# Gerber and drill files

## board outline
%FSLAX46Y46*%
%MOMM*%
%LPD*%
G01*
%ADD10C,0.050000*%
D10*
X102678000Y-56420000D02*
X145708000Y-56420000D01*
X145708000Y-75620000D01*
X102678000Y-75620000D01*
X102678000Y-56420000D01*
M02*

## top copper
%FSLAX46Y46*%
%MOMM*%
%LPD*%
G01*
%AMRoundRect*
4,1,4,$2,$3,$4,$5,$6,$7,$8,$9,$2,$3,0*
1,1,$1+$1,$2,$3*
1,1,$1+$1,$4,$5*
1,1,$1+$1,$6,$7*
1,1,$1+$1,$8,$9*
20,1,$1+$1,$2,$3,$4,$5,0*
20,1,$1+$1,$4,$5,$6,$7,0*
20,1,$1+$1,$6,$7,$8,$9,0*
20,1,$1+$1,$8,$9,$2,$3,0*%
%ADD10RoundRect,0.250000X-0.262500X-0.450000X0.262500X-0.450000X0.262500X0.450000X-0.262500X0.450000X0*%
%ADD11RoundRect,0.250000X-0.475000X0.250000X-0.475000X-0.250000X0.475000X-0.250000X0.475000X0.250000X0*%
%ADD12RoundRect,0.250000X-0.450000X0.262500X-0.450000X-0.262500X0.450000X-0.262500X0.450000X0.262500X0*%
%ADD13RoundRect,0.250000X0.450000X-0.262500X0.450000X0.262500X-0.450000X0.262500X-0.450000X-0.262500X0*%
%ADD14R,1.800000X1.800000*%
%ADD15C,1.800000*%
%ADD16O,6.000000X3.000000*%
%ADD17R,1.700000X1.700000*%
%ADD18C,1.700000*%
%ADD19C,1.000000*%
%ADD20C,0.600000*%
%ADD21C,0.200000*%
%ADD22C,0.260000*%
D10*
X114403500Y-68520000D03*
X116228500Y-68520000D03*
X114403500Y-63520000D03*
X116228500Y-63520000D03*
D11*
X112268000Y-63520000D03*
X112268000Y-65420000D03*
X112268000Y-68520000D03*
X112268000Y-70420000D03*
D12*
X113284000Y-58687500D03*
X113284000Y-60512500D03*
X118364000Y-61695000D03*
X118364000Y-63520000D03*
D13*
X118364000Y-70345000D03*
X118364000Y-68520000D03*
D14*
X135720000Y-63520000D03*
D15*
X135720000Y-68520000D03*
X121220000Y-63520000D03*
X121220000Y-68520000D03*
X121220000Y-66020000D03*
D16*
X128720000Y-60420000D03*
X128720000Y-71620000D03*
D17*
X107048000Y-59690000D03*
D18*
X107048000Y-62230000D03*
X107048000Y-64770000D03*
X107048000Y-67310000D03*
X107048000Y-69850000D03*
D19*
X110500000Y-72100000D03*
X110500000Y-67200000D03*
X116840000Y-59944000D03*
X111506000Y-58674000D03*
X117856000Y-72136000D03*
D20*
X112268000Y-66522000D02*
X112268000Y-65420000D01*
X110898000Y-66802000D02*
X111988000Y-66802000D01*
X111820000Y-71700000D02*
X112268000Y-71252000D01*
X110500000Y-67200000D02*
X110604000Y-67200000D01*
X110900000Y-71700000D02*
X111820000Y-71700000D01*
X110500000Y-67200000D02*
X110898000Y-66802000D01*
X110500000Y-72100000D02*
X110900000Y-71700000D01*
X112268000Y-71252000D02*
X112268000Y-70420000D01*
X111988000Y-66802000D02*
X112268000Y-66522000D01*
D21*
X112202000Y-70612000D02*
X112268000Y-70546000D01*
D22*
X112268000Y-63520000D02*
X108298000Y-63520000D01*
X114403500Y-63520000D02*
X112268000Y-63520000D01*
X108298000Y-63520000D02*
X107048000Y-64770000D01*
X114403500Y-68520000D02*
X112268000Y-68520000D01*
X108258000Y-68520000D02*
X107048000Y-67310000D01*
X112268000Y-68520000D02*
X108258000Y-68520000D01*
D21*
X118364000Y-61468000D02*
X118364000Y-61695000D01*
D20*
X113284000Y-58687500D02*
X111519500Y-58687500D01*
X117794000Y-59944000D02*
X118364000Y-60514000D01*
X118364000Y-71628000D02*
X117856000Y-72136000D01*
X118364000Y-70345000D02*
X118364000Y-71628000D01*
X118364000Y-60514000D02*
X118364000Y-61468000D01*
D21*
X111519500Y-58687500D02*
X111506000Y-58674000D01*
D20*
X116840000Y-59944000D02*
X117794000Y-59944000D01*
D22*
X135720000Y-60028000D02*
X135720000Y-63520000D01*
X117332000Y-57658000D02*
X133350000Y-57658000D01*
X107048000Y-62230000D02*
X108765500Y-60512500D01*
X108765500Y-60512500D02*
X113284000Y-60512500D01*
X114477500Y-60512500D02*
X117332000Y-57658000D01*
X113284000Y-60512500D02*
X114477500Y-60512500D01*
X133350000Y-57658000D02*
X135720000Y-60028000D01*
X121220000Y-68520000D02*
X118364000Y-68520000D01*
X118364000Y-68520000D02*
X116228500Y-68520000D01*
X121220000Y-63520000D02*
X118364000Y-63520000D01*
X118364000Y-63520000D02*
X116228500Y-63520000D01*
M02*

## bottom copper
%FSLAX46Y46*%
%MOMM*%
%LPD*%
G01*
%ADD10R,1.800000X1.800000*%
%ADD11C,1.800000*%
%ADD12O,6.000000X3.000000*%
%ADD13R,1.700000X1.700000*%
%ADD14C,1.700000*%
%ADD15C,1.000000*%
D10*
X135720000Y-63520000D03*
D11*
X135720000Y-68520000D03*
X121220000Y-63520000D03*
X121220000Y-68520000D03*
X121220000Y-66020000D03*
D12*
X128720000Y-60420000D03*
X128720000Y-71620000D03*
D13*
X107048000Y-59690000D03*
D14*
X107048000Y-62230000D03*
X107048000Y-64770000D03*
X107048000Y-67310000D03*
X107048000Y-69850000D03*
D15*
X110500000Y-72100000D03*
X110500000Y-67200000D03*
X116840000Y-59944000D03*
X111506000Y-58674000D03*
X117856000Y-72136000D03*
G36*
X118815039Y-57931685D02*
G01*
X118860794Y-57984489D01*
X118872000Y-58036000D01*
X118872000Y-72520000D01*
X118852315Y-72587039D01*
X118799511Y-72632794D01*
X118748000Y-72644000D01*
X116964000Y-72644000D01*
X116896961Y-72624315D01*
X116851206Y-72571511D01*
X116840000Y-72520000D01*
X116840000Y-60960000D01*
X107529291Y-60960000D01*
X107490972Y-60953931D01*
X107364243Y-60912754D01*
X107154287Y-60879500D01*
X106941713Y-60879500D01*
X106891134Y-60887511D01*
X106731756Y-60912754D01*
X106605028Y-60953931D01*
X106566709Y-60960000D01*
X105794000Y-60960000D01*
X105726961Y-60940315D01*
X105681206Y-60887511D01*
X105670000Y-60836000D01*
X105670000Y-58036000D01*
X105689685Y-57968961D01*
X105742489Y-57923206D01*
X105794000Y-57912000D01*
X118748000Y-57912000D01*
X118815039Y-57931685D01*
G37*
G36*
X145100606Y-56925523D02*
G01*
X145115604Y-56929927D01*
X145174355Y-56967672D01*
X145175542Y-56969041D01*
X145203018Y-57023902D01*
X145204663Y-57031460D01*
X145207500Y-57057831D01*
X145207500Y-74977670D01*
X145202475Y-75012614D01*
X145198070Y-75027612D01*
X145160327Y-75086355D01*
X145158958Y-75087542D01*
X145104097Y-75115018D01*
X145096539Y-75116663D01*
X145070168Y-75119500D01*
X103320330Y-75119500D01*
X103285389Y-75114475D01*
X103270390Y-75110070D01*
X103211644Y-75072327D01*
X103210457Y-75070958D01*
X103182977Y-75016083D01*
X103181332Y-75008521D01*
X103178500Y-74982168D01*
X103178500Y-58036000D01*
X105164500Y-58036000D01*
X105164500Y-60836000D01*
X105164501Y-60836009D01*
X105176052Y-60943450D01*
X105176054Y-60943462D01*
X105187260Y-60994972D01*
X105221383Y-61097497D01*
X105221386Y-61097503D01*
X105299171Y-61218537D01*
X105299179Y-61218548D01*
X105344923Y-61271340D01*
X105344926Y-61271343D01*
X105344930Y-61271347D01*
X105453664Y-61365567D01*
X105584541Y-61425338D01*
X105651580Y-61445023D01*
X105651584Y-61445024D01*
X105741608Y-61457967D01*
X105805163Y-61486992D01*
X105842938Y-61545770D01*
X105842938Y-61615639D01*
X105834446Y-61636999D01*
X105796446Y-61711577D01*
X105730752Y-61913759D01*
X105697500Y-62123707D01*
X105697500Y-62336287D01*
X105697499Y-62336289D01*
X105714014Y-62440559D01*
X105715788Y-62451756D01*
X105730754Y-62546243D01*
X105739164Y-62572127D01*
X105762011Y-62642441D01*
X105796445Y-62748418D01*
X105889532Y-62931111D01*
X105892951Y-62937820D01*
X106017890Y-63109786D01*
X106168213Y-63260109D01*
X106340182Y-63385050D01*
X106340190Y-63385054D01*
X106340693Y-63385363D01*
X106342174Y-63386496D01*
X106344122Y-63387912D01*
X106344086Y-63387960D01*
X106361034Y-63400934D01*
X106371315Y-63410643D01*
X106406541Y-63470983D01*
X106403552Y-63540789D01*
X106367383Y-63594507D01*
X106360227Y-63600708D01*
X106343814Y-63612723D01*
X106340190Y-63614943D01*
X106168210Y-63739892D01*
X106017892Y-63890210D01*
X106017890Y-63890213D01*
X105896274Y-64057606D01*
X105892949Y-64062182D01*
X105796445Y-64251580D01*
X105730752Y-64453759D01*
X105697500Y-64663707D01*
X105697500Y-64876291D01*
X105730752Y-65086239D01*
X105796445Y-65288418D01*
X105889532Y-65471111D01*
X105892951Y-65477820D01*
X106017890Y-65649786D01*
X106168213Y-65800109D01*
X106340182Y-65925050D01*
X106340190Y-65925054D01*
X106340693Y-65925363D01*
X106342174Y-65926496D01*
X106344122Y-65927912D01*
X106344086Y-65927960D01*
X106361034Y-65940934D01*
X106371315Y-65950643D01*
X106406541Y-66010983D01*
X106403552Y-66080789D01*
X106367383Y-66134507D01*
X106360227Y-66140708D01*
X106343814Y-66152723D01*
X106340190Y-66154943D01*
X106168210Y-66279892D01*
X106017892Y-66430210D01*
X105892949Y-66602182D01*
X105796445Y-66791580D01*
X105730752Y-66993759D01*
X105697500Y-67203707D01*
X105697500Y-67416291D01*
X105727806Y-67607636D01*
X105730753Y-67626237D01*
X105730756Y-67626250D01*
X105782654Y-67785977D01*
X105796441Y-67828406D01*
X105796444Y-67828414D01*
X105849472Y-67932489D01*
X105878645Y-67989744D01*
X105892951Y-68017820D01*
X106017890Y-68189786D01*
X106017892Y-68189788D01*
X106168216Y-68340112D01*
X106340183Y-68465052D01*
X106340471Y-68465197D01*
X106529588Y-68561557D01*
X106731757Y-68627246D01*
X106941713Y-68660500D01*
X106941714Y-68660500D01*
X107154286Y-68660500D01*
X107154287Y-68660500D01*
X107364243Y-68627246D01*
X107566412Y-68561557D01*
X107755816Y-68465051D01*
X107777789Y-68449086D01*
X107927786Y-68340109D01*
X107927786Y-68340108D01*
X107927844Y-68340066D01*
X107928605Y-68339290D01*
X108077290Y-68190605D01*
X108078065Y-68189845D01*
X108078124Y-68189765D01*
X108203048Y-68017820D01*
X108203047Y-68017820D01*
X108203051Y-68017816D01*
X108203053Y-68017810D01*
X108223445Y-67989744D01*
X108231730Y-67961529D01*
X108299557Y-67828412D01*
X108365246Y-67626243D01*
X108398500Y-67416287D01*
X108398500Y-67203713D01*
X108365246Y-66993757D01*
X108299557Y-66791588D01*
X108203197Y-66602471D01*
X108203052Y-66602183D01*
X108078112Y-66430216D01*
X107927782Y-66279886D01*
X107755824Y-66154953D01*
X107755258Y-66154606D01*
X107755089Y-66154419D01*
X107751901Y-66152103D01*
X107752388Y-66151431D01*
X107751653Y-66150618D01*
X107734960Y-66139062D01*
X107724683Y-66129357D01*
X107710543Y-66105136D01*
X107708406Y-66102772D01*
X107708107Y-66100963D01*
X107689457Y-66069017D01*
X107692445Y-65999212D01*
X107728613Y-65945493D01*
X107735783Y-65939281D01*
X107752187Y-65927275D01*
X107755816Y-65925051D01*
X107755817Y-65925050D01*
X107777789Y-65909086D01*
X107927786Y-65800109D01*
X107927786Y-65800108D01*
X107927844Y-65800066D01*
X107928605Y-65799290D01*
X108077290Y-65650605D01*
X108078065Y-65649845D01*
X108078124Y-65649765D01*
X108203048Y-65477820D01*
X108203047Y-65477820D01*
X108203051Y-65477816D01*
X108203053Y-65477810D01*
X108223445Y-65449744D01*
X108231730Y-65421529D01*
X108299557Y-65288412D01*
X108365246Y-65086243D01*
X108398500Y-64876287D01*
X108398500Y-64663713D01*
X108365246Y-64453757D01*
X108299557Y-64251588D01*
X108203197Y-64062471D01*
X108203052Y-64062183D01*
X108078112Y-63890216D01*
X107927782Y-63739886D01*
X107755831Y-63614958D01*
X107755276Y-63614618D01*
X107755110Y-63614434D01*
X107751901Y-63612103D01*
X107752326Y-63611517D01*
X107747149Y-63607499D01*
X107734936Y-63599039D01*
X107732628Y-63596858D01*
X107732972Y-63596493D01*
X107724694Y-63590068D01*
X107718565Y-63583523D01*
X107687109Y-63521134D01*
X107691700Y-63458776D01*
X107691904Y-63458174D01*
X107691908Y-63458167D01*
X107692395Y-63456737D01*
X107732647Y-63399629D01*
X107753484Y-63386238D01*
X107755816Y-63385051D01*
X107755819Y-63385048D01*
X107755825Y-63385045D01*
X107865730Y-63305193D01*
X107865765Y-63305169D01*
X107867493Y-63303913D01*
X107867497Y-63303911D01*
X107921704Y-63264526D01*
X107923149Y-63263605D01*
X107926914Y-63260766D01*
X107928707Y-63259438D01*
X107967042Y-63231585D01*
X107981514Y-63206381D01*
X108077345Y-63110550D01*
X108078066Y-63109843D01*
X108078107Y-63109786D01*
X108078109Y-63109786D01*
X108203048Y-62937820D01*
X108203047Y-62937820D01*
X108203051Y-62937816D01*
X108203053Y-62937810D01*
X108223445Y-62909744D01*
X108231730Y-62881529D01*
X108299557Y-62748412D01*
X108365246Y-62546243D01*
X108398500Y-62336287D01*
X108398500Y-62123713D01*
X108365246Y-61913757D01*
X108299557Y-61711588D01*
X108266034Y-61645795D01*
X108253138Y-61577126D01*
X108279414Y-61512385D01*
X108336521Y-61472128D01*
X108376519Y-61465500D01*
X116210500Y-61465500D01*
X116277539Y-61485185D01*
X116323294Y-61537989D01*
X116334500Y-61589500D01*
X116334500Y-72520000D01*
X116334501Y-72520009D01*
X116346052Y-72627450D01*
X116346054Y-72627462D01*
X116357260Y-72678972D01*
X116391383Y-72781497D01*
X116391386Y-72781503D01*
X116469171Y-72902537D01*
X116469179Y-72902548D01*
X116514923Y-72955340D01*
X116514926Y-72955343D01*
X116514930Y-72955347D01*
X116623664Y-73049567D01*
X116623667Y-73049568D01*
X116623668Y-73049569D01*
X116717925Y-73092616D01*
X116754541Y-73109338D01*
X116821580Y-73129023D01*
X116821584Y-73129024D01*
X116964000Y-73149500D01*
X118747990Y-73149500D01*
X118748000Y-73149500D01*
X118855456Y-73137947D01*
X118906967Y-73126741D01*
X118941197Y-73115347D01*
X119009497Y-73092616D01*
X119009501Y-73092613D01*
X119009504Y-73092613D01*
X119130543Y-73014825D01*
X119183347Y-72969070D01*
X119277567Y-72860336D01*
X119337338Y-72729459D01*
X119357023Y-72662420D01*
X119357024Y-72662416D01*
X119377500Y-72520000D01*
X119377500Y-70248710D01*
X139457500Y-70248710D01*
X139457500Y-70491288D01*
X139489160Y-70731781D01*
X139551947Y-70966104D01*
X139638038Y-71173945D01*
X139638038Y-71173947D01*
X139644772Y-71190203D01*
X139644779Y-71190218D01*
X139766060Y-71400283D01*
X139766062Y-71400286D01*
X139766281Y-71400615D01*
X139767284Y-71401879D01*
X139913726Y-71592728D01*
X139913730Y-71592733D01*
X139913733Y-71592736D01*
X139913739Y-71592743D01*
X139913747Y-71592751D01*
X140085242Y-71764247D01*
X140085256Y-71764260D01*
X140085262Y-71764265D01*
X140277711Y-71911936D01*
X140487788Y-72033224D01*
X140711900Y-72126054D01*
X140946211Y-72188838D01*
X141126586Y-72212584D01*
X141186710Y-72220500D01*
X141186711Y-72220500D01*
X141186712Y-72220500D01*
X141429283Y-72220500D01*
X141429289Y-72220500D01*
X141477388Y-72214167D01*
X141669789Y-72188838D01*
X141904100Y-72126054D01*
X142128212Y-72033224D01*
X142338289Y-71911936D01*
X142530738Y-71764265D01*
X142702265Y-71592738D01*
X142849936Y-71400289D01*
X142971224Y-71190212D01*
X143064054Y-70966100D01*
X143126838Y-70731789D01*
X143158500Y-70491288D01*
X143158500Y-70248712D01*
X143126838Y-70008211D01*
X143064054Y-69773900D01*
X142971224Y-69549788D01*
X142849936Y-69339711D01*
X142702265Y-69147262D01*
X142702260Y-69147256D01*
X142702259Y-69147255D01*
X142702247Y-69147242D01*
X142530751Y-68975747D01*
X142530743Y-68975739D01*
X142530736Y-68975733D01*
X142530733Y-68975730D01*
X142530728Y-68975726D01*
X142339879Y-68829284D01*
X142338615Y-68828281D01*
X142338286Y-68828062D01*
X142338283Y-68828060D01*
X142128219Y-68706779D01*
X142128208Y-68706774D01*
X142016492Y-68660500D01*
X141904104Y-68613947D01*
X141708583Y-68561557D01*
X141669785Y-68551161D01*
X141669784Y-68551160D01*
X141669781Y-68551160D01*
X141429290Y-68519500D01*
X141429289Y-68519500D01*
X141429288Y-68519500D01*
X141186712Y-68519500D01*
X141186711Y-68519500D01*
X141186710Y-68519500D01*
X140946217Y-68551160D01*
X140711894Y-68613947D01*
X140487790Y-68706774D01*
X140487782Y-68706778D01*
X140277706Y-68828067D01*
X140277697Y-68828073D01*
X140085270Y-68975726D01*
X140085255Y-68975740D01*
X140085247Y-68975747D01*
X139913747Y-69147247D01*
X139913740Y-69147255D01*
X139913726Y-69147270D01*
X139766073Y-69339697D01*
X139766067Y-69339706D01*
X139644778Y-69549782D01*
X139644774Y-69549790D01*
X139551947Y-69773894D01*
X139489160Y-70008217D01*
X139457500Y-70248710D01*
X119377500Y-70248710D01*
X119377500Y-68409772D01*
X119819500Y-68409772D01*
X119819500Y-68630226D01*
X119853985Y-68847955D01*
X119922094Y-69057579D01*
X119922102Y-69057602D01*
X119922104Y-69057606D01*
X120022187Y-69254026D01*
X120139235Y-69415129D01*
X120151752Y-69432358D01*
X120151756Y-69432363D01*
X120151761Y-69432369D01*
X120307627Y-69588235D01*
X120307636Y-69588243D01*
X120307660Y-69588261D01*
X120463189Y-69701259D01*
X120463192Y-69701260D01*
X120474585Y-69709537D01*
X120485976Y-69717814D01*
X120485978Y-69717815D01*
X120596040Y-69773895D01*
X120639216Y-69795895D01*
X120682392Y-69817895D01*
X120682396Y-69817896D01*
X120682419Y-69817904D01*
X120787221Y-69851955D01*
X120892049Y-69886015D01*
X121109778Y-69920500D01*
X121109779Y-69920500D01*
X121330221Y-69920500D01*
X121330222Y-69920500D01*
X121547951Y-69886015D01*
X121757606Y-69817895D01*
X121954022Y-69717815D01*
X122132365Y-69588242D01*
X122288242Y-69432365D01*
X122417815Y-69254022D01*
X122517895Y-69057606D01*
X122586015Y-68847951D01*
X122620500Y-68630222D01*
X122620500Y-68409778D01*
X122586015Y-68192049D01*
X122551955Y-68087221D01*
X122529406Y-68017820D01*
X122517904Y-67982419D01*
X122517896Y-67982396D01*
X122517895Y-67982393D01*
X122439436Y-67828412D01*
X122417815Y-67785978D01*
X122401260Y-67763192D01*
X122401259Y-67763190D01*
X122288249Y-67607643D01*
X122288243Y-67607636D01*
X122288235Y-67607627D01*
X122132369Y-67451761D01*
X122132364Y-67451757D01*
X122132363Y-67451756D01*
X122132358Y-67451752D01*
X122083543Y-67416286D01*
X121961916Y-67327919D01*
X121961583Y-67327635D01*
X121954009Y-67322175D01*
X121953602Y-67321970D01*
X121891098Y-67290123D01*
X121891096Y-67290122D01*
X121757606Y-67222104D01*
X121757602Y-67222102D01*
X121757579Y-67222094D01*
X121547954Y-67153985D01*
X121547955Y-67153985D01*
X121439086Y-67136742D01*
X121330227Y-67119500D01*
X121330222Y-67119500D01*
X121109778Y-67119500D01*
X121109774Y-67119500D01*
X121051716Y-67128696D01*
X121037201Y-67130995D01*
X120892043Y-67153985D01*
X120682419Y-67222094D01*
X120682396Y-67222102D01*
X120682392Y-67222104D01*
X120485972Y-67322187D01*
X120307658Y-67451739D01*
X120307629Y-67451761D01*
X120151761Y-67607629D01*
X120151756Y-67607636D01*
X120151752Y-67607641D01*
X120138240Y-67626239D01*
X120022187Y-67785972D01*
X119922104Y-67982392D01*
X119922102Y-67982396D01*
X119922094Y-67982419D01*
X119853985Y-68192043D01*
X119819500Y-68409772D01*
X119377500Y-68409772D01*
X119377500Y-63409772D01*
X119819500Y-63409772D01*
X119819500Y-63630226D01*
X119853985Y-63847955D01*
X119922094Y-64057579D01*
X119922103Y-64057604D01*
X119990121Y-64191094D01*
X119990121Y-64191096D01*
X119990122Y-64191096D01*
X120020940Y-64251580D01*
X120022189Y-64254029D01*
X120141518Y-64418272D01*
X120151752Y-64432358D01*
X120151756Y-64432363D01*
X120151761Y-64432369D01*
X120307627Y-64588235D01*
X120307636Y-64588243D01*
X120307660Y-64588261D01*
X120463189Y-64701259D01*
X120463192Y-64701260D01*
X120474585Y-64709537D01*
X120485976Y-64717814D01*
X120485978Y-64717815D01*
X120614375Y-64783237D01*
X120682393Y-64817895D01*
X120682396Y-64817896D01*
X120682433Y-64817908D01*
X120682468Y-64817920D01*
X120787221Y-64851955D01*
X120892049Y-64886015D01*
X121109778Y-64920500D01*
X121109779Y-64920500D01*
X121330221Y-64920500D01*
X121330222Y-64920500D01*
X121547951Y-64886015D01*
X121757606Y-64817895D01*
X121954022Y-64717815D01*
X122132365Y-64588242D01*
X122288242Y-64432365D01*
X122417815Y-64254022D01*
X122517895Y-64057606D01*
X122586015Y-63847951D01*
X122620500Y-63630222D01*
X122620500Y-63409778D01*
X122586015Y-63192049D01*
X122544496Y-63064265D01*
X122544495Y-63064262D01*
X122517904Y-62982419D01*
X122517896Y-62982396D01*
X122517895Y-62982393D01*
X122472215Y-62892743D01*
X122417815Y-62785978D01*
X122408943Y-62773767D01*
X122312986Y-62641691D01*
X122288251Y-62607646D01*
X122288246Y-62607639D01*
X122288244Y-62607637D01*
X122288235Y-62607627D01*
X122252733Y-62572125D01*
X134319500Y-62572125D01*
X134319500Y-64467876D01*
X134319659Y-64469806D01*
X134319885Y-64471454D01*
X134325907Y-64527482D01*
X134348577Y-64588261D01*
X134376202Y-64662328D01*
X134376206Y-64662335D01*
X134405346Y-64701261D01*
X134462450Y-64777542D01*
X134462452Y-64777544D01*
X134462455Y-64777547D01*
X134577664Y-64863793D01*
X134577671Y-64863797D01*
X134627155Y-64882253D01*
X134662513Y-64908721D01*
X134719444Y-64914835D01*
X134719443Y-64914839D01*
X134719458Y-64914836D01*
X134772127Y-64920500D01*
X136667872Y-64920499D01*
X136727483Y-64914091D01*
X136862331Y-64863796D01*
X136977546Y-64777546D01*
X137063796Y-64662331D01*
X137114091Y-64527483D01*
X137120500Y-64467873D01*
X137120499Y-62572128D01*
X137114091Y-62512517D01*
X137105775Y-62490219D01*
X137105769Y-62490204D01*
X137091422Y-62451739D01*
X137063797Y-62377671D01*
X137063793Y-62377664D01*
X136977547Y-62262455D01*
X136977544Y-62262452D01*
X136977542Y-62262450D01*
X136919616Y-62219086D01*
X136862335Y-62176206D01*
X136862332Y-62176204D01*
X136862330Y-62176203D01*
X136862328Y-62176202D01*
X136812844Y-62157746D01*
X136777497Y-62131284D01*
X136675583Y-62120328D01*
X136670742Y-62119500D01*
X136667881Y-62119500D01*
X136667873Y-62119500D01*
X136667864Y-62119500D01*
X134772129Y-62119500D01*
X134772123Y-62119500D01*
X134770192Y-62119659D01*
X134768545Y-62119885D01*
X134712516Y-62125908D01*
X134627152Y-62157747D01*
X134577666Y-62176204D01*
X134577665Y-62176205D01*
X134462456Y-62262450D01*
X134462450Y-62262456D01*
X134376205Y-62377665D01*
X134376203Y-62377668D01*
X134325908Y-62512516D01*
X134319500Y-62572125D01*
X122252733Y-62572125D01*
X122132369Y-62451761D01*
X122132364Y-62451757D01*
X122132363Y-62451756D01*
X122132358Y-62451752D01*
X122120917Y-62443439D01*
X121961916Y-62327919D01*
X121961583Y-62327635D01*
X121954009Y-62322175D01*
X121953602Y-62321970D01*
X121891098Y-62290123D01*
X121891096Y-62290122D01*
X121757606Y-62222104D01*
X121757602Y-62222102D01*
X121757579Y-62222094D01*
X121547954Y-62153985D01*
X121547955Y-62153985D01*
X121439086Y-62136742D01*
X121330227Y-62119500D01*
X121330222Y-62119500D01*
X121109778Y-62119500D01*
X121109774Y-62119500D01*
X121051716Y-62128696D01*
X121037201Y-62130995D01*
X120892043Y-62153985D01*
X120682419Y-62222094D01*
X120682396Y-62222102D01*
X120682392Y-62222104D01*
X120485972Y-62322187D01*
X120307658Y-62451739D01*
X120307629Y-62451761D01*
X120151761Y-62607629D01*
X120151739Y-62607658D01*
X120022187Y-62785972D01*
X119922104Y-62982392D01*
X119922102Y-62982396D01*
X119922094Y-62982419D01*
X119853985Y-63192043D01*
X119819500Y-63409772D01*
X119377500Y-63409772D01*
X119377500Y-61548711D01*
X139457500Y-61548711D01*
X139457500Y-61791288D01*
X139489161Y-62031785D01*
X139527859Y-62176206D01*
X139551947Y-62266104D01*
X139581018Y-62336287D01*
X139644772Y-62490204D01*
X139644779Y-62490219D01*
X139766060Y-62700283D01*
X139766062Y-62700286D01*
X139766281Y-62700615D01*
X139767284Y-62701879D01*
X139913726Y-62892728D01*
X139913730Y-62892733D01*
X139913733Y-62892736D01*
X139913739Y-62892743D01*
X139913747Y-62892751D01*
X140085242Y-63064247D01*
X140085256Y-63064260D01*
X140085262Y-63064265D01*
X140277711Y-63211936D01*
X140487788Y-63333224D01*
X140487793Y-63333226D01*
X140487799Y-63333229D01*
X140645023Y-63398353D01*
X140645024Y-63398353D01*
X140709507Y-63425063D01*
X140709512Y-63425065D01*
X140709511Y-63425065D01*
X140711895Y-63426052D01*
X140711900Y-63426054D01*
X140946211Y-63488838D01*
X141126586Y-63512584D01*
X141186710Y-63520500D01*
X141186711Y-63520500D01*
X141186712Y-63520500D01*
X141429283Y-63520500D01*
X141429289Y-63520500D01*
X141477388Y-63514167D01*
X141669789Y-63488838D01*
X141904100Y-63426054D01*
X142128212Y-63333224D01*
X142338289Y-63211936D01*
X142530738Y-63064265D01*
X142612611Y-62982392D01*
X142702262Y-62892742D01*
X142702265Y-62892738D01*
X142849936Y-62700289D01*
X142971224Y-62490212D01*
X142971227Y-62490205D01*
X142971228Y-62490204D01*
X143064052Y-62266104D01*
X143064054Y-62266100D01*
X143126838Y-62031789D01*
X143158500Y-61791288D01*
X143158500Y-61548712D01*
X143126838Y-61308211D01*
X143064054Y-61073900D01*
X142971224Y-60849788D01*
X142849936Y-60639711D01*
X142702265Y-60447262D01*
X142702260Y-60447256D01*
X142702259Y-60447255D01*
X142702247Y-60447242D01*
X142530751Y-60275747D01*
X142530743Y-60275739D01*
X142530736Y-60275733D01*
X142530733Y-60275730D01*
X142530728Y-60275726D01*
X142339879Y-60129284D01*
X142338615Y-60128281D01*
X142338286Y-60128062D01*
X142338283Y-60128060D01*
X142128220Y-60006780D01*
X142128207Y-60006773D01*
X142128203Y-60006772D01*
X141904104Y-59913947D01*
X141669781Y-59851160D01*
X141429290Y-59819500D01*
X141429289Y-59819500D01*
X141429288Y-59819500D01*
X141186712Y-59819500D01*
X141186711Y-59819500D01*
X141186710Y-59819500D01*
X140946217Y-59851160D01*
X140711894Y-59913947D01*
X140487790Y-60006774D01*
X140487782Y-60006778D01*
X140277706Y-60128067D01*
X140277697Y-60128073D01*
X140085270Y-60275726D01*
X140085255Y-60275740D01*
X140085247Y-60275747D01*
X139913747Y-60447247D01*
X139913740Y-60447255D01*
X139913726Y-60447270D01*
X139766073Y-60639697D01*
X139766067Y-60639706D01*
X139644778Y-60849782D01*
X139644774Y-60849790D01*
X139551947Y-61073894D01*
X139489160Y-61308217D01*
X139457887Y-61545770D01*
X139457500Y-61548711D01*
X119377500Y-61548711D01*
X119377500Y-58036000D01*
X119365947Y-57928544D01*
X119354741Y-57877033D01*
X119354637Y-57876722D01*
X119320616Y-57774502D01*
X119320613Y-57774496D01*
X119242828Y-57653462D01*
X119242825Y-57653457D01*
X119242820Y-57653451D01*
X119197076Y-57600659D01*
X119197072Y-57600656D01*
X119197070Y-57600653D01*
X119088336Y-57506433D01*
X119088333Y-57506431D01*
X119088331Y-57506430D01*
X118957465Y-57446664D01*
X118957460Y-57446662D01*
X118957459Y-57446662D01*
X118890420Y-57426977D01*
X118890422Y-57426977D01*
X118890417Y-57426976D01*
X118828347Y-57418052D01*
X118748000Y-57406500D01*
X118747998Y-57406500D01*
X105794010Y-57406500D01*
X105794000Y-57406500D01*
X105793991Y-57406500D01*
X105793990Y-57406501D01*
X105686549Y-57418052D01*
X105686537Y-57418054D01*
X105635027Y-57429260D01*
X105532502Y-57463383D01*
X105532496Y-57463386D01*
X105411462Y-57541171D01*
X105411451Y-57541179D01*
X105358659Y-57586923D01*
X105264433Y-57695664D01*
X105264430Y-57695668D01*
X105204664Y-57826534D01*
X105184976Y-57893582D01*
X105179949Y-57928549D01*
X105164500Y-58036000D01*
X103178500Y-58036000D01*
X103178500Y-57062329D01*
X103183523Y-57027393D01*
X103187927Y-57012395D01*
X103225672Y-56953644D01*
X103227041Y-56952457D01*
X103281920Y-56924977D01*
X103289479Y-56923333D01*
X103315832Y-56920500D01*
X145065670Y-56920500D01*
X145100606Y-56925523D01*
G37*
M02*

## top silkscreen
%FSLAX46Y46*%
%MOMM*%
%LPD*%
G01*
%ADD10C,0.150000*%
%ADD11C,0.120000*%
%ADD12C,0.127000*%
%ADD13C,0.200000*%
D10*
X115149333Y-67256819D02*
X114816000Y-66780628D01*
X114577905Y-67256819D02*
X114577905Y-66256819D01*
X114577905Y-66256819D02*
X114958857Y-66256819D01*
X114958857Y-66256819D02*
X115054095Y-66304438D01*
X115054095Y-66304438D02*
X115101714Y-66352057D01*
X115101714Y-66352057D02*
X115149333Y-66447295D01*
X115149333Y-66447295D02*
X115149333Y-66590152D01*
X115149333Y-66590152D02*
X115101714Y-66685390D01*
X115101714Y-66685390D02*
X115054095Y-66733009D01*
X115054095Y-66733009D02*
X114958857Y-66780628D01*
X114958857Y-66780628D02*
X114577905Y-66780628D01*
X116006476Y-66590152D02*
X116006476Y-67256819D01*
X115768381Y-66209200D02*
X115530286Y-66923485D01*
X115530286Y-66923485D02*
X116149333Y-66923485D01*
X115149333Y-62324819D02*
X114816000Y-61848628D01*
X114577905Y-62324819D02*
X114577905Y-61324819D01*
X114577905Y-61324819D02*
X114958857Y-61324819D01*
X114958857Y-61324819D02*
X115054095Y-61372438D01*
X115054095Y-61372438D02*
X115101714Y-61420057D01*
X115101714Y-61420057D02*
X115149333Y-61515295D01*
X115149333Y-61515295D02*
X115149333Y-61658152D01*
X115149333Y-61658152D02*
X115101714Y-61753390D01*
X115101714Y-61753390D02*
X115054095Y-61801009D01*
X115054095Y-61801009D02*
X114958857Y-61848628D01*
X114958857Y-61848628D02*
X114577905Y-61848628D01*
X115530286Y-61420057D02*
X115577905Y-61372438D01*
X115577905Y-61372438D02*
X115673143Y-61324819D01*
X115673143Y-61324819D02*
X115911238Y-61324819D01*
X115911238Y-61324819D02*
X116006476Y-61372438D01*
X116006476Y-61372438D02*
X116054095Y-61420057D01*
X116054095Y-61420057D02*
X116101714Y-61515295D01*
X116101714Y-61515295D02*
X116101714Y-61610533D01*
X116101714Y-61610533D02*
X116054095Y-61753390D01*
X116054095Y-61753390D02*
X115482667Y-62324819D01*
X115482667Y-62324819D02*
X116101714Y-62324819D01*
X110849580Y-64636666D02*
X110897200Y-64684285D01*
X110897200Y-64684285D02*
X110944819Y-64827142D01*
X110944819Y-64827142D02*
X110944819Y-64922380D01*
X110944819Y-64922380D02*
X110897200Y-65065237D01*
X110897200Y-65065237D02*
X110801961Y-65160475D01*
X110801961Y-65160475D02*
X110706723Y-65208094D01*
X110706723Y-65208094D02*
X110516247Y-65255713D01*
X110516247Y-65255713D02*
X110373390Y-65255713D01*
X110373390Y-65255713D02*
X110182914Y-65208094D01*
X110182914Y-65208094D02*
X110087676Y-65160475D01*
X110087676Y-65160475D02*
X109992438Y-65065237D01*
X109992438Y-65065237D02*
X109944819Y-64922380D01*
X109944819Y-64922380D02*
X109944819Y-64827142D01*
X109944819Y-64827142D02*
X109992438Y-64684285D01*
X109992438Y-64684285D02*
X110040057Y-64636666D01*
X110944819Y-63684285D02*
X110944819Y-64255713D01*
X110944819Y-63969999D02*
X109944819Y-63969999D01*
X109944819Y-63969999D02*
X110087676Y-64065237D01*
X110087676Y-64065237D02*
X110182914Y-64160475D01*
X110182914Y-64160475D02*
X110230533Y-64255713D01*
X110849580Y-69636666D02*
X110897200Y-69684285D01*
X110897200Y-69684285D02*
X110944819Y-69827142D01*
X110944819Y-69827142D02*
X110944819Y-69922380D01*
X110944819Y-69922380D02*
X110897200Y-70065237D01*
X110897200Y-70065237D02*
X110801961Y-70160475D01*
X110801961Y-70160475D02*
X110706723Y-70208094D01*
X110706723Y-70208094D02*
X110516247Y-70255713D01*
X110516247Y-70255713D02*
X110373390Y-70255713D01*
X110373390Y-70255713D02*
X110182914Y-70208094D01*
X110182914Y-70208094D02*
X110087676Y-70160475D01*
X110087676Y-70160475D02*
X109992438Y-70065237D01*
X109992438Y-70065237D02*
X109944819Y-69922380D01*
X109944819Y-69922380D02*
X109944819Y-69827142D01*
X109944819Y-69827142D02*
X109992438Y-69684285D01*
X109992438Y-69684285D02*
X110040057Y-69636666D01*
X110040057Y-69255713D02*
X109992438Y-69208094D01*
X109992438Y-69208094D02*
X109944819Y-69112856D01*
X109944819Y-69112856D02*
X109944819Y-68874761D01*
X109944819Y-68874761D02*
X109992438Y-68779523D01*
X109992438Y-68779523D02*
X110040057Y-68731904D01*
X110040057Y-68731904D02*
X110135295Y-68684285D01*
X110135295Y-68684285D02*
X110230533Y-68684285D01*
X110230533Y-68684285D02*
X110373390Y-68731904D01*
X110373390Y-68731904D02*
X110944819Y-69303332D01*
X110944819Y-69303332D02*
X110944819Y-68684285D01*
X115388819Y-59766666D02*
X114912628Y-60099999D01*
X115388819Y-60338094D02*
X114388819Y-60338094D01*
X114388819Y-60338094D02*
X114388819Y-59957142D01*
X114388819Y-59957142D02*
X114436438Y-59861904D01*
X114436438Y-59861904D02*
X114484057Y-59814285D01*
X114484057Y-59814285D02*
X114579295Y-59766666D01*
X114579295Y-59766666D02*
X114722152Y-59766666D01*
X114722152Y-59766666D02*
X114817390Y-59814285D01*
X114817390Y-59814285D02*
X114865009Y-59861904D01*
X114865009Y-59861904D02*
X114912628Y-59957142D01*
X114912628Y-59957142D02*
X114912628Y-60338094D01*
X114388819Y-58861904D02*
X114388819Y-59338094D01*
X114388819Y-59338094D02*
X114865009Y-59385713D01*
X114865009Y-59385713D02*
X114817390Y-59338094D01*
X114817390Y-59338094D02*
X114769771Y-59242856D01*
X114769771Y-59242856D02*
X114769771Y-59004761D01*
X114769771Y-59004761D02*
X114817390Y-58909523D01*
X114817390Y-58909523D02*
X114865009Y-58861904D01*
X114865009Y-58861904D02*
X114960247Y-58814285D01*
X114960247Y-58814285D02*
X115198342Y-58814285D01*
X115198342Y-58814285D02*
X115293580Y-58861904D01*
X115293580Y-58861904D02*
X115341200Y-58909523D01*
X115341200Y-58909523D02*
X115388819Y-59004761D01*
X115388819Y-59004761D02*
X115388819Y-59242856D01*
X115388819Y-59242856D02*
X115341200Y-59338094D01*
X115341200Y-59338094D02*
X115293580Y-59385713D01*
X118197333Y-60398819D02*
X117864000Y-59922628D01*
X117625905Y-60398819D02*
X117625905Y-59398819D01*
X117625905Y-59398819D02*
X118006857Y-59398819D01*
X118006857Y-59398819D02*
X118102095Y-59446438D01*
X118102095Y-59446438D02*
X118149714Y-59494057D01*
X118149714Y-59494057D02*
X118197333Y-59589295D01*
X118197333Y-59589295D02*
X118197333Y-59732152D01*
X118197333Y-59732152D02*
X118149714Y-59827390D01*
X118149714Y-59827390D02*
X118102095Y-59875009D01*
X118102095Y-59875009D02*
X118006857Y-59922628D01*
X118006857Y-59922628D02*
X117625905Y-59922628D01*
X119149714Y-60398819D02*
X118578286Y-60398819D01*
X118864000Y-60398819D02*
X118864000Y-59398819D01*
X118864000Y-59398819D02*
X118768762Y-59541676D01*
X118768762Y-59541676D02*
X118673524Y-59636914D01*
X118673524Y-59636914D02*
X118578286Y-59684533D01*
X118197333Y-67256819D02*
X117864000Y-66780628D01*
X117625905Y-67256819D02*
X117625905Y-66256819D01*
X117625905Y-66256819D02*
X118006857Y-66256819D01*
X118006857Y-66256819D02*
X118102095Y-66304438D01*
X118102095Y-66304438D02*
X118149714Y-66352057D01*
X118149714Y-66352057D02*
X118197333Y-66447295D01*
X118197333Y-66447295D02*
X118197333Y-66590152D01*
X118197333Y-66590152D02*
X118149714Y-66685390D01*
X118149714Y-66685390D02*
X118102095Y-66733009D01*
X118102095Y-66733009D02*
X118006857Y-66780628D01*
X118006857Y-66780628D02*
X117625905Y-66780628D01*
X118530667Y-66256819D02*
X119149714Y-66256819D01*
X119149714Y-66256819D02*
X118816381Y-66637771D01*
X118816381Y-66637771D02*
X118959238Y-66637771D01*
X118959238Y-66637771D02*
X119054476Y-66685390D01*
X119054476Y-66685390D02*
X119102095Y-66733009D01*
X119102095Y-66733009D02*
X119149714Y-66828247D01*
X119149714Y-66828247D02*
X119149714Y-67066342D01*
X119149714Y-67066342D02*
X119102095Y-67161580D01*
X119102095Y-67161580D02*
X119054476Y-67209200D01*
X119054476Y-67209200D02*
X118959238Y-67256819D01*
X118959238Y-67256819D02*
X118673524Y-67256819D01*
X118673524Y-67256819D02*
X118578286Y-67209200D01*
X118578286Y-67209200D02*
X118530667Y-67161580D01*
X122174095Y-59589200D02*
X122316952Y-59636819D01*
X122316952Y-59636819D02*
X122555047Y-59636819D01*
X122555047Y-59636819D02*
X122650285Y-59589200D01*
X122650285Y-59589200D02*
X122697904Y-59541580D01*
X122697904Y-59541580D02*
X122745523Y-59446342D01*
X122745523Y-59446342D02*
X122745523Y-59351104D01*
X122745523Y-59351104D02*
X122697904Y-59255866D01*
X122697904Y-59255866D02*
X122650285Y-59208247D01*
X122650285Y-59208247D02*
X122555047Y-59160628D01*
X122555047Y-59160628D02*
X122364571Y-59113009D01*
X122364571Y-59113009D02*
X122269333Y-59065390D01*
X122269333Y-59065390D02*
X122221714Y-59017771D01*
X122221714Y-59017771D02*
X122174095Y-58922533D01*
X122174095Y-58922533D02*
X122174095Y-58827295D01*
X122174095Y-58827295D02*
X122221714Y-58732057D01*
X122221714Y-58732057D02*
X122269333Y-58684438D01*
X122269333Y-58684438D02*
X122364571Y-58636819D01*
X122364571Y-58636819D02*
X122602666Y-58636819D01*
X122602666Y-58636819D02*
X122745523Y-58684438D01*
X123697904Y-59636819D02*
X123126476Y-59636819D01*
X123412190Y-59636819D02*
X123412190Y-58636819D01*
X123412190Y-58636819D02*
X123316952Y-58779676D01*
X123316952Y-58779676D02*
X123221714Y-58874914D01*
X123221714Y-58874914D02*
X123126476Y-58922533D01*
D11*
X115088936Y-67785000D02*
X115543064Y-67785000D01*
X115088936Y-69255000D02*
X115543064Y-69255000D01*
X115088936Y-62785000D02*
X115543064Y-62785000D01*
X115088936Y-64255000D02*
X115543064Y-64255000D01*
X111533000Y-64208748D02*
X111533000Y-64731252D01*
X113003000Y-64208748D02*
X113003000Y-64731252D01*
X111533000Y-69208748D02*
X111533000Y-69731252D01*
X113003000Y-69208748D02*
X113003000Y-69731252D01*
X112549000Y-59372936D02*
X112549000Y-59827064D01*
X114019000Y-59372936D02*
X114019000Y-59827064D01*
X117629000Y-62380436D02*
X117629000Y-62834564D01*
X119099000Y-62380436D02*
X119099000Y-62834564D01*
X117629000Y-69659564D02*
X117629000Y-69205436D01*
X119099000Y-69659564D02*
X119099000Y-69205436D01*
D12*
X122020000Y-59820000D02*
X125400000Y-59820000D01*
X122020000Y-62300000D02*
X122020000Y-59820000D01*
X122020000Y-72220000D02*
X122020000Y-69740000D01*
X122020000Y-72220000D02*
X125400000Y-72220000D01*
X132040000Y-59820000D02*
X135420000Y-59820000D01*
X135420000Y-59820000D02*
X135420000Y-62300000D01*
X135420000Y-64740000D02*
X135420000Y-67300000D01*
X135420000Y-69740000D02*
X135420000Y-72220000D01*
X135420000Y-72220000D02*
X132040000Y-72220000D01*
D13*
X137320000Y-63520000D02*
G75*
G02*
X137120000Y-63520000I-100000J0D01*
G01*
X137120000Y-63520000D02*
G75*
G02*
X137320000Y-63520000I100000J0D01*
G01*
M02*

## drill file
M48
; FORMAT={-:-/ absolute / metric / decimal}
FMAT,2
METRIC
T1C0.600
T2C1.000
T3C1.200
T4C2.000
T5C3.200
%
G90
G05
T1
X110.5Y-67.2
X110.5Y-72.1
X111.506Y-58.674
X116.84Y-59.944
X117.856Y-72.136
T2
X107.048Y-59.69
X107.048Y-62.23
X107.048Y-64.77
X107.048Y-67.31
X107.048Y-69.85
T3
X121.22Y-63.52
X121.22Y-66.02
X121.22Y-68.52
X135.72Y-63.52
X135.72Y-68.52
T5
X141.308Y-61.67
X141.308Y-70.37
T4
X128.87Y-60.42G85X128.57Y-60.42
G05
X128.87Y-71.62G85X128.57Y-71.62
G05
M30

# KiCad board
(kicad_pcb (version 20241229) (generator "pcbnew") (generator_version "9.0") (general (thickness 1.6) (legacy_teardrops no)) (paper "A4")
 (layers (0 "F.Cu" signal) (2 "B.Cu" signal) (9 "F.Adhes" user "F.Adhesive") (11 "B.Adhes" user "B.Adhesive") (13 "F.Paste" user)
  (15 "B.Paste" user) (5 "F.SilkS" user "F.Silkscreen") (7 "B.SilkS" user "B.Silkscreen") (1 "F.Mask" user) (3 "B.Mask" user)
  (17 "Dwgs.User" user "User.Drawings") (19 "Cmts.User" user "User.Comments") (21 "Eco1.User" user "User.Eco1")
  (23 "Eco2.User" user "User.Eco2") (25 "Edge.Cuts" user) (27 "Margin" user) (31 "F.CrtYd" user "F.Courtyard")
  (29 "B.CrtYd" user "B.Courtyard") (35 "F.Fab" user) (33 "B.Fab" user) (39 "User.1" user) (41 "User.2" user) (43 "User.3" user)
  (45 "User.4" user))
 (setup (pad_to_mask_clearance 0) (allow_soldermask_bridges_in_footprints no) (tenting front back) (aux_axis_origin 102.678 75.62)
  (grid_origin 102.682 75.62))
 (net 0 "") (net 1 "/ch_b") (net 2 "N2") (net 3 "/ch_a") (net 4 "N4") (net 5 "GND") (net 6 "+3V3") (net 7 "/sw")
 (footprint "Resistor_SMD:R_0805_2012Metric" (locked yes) (layer "F.Cu") (at 115.316 68.52)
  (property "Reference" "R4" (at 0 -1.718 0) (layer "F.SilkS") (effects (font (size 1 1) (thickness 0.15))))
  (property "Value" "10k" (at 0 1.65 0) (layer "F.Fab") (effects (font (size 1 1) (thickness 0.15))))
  (fp_line (start -0.227064 -0.735) (end 0.227064 -0.735) (stroke (width 0.12) (type solid)) (layer "F.SilkS"))
  (fp_line (start -0.227064 0.735) (end 0.227064 0.735) (stroke (width 0.12) (type solid)) (layer "F.SilkS"))
  (pad "1" smd roundrect (at -0.9125 0) (size 1.025 1.4) (layers "F.Cu" "F.Mask" "F.Paste") (roundrect_rratio 0.243902) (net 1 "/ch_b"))
  (pad "2" smd roundrect (at 0.9125 0) (size 1.025 1.4) (layers "F.Cu" "F.Mask" "F.Paste") (roundrect_rratio 0.243902) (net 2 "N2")))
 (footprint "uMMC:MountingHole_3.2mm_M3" (layer "F.Cu") (at 141.308 70.37)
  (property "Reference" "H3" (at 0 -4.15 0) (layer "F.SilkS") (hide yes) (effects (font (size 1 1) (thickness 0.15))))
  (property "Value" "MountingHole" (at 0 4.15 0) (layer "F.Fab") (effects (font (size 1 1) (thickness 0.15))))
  (pad "" np_thru_hole circle (at 0 0) (size 3.2 3.2) (drill 3.2) (layers "*.Cu" "*.Mask")))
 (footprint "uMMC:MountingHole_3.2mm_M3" (layer "F.Cu") (at 141.308 61.67)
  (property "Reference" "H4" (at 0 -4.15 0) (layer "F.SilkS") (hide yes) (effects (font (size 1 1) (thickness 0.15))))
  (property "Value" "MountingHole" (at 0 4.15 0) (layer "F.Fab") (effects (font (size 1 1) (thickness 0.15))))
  (pad "" np_thru_hole circle (at 0 0) (size 3.2 3.2) (drill 3.2) (layers "*.Cu" "*.Mask")))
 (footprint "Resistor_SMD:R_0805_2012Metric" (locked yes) (layer "F.Cu") (at 115.316 63.52)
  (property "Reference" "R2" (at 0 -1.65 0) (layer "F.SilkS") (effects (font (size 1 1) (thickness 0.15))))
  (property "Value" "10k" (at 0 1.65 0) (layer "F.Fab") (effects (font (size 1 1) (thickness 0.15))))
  (fp_line (start -0.227064 -0.735) (end 0.227064 -0.735) (stroke (width 0.12) (type solid)) (layer "F.SilkS"))
  (fp_line (start -0.227064 0.735) (end 0.227064 0.735) (stroke (width 0.12) (type solid)) (layer "F.SilkS"))
  (pad "1" smd roundrect (at -0.9125 0) (size 1.025 1.4) (layers "F.Cu" "F.Mask" "F.Paste") (roundrect_rratio 0.243902) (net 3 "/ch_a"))
  (pad "2" smd roundrect (at 0.9125 0) (size 1.025 1.4) (layers "F.Cu" "F.Mask" "F.Paste") (roundrect_rratio 0.243902) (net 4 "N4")))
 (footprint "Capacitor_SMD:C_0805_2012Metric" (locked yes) (layer "F.Cu") (at 112.268 64.47 -90)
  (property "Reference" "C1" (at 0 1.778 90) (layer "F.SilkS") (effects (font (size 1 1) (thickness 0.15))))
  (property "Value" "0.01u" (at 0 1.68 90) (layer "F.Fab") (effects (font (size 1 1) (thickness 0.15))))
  (fp_line (start -0.261252 0.735) (end 0.261252 0.735) (stroke (width 0.12) (type solid)) (layer "F.SilkS"))
  (fp_line (start -0.261252 -0.735) (end 0.261252 -0.735) (stroke (width 0.12) (type solid)) (layer "F.SilkS"))
  (pad "1" smd roundrect (at -0.95 0 270) (size 1 1.45) (layers "F.Cu" "F.Mask" "F.Paste") (roundrect_rratio 0.25) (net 3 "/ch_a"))
  (pad "2" smd roundrect (at 0.95 0 270) (size 1 1.45) (layers "F.Cu" "F.Mask" "F.Paste") (roundrect_rratio 0.25) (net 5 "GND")))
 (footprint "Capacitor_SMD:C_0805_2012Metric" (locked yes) (layer "F.Cu") (at 112.268 69.47 -90)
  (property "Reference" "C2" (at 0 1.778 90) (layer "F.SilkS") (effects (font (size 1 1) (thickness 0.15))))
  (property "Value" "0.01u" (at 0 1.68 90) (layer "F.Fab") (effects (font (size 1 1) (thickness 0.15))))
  (fp_line (start -0.261252 0.735) (end 0.261252 0.735) (stroke (width 0.12) (type solid)) (layer "F.SilkS"))
  (fp_line (start -0.261252 -0.735) (end 0.261252 -0.735) (stroke (width 0.12) (type solid)) (layer "F.SilkS"))
  (pad "1" smd roundrect (at -0.95 0 270) (size 1 1.45) (layers "F.Cu" "F.Mask" "F.Paste") (roundrect_rratio 0.25) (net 1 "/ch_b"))
  (pad "2" smd roundrect (at 0.95 0 270) (size 1 1.45) (layers "F.Cu" "F.Mask" "F.Paste") (roundrect_rratio 0.25) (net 5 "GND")))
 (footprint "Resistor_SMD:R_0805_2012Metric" (layer "F.Cu") (at 113.284 59.6 -90)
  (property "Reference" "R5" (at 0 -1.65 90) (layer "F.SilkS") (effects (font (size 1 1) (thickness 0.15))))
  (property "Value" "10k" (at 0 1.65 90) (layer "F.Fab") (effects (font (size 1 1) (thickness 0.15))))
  (fp_line (start -0.227064 0.735) (end 0.227064 0.735) (stroke (width 0.12) (type solid)) (layer "F.SilkS"))
  (fp_line (start -0.227064 -0.735) (end 0.227064 -0.735) (stroke (width 0.12) (type solid)) (layer "F.SilkS"))
  (pad "1" smd roundrect (at -0.9125 0 270) (size 1.025 1.4) (layers "F.Cu" "F.Mask" "F.Paste") (roundrect_rratio 0.243902) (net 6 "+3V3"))
  (pad "2" smd roundrect (at 0.9125 0 270) (size 1.025 1.4) (layers "F.Cu" "F.Mask" "F.Paste") (roundrect_rratio 0.243902) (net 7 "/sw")))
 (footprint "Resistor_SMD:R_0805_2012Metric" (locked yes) (layer "F.Cu") (at 118.364 62.6075 -90)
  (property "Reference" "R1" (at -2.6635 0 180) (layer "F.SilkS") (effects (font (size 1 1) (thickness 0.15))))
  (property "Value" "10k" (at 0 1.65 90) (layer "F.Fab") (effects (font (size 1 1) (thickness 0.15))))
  (fp_line (start -0.227064 0.735) (end 0.227064 0.735) (stroke (width 0.12) (type solid)) (layer "F.SilkS"))
  (fp_line (start -0.227064 -0.735) (end 0.227064 -0.735) (stroke (width 0.12) (type solid)) (layer "F.SilkS"))
  (pad "1" smd roundrect (at -0.9125 0 270) (size 1.025 1.4) (layers "F.Cu" "F.Mask" "F.Paste") (roundrect_rratio 0.243902) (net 6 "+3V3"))
  (pad "2" smd roundrect (at 0.9125 0 270) (size 1.025 1.4) (layers "F.Cu" "F.Mask" "F.Paste") (roundrect_rratio 0.243902) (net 4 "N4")))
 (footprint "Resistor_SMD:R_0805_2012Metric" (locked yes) (layer "F.Cu") (at 118.364 69.4325 90)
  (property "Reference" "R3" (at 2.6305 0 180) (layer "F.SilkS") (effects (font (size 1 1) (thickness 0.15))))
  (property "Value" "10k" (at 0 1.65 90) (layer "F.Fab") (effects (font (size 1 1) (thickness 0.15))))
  (fp_line (start -0.227064 -0.735) (end 0.227064 -0.735) (stroke (width 0.12) (type solid)) (layer "F.SilkS"))
  (fp_line (start -0.227064 0.735) (end 0.227064 0.735) (stroke (width 0.12) (type solid)) (layer "F.SilkS"))
  (pad "1" smd roundrect (at -0.9125 0 90) (size 1.025 1.4) (layers "F.Cu" "F.Mask" "F.Paste") (roundrect_rratio 0.243902) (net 6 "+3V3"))
  (pad "2" smd roundrect (at 0.9125 0 90) (size 1.025 1.4) (layers "F.Cu" "F.Mask" "F.Paste") (roundrect_rratio 0.243902) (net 2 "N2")))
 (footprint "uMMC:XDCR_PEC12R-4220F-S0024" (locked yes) (layer "F.Cu") (at 128.72 66.02 -90)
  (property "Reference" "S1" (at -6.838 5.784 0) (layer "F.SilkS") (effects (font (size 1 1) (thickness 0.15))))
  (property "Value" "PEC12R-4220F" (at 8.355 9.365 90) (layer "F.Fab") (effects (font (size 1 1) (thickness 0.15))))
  (fp_line (start -6.2 6.7) (end -6.2 3.32) (stroke (width 0.127) (type solid)) (layer "F.SilkS"))
  (fp_line (start -3.72 6.7) (end -6.2 6.7) (stroke (width 0.127) (type solid)) (layer "F.SilkS"))
  (fp_line (start 6.2 6.7) (end 3.72 6.7) (stroke (width 0.127) (type solid)) (layer "F.SilkS"))
  (fp_line (start 6.2 6.7) (end 6.2 3.32) (stroke (width 0.127) (type solid)) (layer "F.SilkS"))
  (fp_line (start -6.2 -3.32) (end -6.2 -6.7) (stroke (width 0.127) (type solid)) (layer "F.SilkS"))
  (fp_line (start -6.2 -6.7) (end -3.72 -6.7) (stroke (width 0.127) (type solid)) (layer "F.SilkS"))
  (fp_line (start -1.28 -6.7) (end 1.28 -6.7) (stroke (width 0.127) (type solid)) (layer "F.SilkS"))
  (fp_line (start 3.72 -6.7) (end 6.2 -6.7) (stroke (width 0.127) (type solid)) (layer "F.SilkS"))
  (fp_line (start 6.2 -6.7) (end 6.2 -3.32) (stroke (width 0.127) (type solid)) (layer "F.SilkS"))
  (fp_circle (center -2.5 -8.5) (end -2.4 -8.5) (stroke (width 0.2) (type solid)) (fill no) (layer "F.SilkS"))
  (pad "1" thru_hole rect (at -2.5 -7 270) (size 1.8 1.8) (drill 1.2) (layers "*.Cu" "*.Mask") (remove_unused_layers no) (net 7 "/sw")
   (solder_mask_margin 0.102))
  (pad "2" thru_hole circle (at 2.5 -7 270) (size 1.8 1.8) (drill 1.2) (layers "*.Cu" "*.Mask") (remove_unused_layers no) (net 5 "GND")
   (solder_mask_margin 0.102))
  (pad "A" thru_hole circle (at -2.5 7.5 270) (size 1.8 1.8) (drill 1.2) (layers "*.Cu" "*.Mask") (remove_unused_layers no) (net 4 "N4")
   (solder_mask_margin 0.102))
  (pad "B" thru_hole circle (at 2.5 7.5 270) (size 1.8 1.8) (drill 1.2) (layers "*.Cu" "*.Mask") (remove_unused_layers no) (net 2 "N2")
   (solder_mask_margin 0.102))
  (pad "C" thru_hole circle (at 0 7.5 270) (size 1.8 1.8) (drill 1.2) (layers "*.Cu" "*.Mask") (remove_unused_layers no) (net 5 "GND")
   (solder_mask_margin 0.102))
  (pad "SH1" thru_hole oval (at -5.6 0 270) (size 3 6) (drill oval 2 2.3) (layers "*.Cu" "*.Mask") (remove_unused_layers no) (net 5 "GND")
   (solder_mask_margin 0.102))
  (pad "SH2" thru_hole oval (at 5.6 0 270) (size 3 6) (drill oval 2 2.3) (layers "*.Cu" "*.Mask") (remove_unused_layers no) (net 5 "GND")
   (solder_mask_margin 0.102)))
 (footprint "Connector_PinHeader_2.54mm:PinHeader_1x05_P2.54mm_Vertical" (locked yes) (layer "B.Cu") (at 107.048 59.69 180)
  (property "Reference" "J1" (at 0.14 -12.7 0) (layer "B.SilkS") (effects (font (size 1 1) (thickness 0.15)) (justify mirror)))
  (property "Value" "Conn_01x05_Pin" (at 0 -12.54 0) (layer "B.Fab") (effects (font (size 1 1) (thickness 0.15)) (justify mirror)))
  (pad "1" thru_hole rect (at 0 0 180) (size 1.7 1.7) (drill 1) (layers "*.Cu" "*.Mask") (remove_unused_layers no) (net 6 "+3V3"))
  (pad "2" thru_hole circle (at 0 -2.54 180) (size 1.7 1.7) (drill 1) (layers "*.Cu" "*.Mask") (remove_unused_layers no) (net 7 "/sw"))
  (pad "3" thru_hole circle (at 0 -5.08 180) (size 1.7 1.7) (drill 1) (layers "*.Cu" "*.Mask") (remove_unused_layers no) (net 3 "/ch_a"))
  (pad "4" thru_hole circle (at 0 -7.62 180) (size 1.7 1.7) (drill 1) (layers "*.Cu" "*.Mask") (remove_unused_layers no) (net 1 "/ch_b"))
  (pad "5" thru_hole circle (at 0 -10.16 180) (size 1.7 1.7) (drill 1) (layers "*.Cu" "*.Mask") (remove_unused_layers no) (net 5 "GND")))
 (gr_rect (start 102.678 56.42) (end 145.708 75.62) (stroke (width 0.05) (type solid)) (fill no) (layer "Edge.Cuts"))
 (segment (start 112.268 66.522) (end 112.268 65.42) (width 0.6) (layer "F.Cu") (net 5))
 (segment (start 110.898 66.802) (end 111.988 66.802) (width 0.6) (layer "F.Cu") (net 5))
 (segment (start 111.82 71.7) (end 112.268 71.252) (width 0.6) (layer "F.Cu") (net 5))
 (segment (start 110.5 67.2) (end 110.604 67.2) (width 0.6) (layer "F.Cu") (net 5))
 (segment (start 110.9 71.7) (end 111.82 71.7) (width 0.6) (layer "F.Cu") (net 5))
 (segment (start 110.5 67.2) (end 110.898 66.802) (width 0.6) (layer "F.Cu") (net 5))
 (segment (start 110.5 72.1) (end 110.9 71.7) (width 0.6) (layer "F.Cu") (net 5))
 (segment (start 112.268 71.252) (end 112.268 70.42) (width 0.6) (layer "F.Cu") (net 5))
 (segment (start 111.988 66.802) (end 112.268 66.522) (width 0.6) (layer "F.Cu") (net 5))
 (segment (start 112.202 70.612) (end 112.268 70.546) (width 0.2) (layer "F.Cu") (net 5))
 (via (at 110.5 72.1) (size 1) (drill 0.6) (layers "F.Cu" "B.Cu") (free yes) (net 5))
 (via (at 110.5 67.2) (size 1) (drill 0.6) (layers "F.Cu" "B.Cu") (free yes) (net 5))
 (segment (start 112.268 63.52) (end 108.298 63.52) (width 0.26) (layer "F.Cu") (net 3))
 (segment (start 114.4035 63.52) (end 112.268 63.52) (width 0.26) (layer "F.Cu") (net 3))
 (segment (start 108.298 63.52) (end 107.048 64.77) (width 0.26) (layer "F.Cu") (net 3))
 (segment (start 114.4035 68.52) (end 112.268 68.52) (width 0.26) (layer "F.Cu") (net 1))
 (segment (start 108.258 68.52) (end 107.048 67.31) (width 0.26) (layer "F.Cu") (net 1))
 (segment (start 112.268 68.52) (end 108.258 68.52) (width 0.26) (layer "F.Cu") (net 1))
 (segment (start 118.364 61.468) (end 118.364 61.695) (width 0.2) (layer "F.Cu") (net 6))
 (segment (start 113.284 58.6875) (end 111.5195 58.6875) (width 0.6) (layer "F.Cu") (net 6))
 (segment (start 117.794 59.944) (end 118.364 60.514) (width 0.6) (layer "F.Cu") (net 6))
 (segment (start 118.364 71.628) (end 117.856 72.136) (width 0.6) (layer "F.Cu") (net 6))
 (segment (start 118.364 70.345) (end 118.364 71.628) (width 0.6) (layer "F.Cu") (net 6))
 (segment (start 118.364 60.514) (end 118.364 61.468) (width 0.6) (layer "F.Cu") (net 6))
 (segment (start 111.5195 58.6875) (end 111.506 58.674) (width 0.2) (layer "F.Cu") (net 6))
 (segment (start 116.84 59.944) (end 117.794 59.944) (width 0.6) (layer "F.Cu") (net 6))
 (via (at 116.84 59.944) (size 1) (drill 0.6) (layers "F.Cu" "B.Cu") (free yes) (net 6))
 (via (at 111.506 58.674) (size 1) (drill 0.6) (layers "F.Cu" "B.Cu") (free yes) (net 6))
 (via (at 117.856 72.136) (size 1) (drill 0.6) (layers "F.Cu" "B.Cu") (free yes) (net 6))
 (segment (start 135.72 60.028) (end 135.72 63.52) (width 0.26) (layer "F.Cu") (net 7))
 (segment (start 117.332 57.658) (end 133.35 57.658) (width 0.26) (layer "F.Cu") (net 7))
 (segment (start 107.048 62.23) (end 108.7655 60.5125) (width 0.26) (layer "F.Cu") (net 7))
 (segment (start 108.7655 60.5125) (end 113.284 60.5125) (width 0.26) (layer "F.Cu") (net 7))
 (segment (start 114.4775 60.5125) (end 117.332 57.658) (width 0.26) (layer "F.Cu") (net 7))
 (segment (start 113.284 60.5125) (end 114.4775 60.5125) (width 0.26) (layer "F.Cu") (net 7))
 (segment (start 133.35 57.658) (end 135.72 60.028) (width 0.26) (layer "F.Cu") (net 7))
 (segment (start 121.22 68.52) (end 118.364 68.52) (width 0.26) (layer "F.Cu") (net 2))
 (segment (start 118.364 68.52) (end 116.2285 68.52) (width 0.26) (layer "F.Cu") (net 2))
 (segment (start 121.22 63.52) (end 118.364 63.52) (width 0.26) (layer "F.Cu") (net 4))
 (segment (start 118.364 63.52) (end 116.2285 63.52) (width 0.26) (layer "F.Cu") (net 4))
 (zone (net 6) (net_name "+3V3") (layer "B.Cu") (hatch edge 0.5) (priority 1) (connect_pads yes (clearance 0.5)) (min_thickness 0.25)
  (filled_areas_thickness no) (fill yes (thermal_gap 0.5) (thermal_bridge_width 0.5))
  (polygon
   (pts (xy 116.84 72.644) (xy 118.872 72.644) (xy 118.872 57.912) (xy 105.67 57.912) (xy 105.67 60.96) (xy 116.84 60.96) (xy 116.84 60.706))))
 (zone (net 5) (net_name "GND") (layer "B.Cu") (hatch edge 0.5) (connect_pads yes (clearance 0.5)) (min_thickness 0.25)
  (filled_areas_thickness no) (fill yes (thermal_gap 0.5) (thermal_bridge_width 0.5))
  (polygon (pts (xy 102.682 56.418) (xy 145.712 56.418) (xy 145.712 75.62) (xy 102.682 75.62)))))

